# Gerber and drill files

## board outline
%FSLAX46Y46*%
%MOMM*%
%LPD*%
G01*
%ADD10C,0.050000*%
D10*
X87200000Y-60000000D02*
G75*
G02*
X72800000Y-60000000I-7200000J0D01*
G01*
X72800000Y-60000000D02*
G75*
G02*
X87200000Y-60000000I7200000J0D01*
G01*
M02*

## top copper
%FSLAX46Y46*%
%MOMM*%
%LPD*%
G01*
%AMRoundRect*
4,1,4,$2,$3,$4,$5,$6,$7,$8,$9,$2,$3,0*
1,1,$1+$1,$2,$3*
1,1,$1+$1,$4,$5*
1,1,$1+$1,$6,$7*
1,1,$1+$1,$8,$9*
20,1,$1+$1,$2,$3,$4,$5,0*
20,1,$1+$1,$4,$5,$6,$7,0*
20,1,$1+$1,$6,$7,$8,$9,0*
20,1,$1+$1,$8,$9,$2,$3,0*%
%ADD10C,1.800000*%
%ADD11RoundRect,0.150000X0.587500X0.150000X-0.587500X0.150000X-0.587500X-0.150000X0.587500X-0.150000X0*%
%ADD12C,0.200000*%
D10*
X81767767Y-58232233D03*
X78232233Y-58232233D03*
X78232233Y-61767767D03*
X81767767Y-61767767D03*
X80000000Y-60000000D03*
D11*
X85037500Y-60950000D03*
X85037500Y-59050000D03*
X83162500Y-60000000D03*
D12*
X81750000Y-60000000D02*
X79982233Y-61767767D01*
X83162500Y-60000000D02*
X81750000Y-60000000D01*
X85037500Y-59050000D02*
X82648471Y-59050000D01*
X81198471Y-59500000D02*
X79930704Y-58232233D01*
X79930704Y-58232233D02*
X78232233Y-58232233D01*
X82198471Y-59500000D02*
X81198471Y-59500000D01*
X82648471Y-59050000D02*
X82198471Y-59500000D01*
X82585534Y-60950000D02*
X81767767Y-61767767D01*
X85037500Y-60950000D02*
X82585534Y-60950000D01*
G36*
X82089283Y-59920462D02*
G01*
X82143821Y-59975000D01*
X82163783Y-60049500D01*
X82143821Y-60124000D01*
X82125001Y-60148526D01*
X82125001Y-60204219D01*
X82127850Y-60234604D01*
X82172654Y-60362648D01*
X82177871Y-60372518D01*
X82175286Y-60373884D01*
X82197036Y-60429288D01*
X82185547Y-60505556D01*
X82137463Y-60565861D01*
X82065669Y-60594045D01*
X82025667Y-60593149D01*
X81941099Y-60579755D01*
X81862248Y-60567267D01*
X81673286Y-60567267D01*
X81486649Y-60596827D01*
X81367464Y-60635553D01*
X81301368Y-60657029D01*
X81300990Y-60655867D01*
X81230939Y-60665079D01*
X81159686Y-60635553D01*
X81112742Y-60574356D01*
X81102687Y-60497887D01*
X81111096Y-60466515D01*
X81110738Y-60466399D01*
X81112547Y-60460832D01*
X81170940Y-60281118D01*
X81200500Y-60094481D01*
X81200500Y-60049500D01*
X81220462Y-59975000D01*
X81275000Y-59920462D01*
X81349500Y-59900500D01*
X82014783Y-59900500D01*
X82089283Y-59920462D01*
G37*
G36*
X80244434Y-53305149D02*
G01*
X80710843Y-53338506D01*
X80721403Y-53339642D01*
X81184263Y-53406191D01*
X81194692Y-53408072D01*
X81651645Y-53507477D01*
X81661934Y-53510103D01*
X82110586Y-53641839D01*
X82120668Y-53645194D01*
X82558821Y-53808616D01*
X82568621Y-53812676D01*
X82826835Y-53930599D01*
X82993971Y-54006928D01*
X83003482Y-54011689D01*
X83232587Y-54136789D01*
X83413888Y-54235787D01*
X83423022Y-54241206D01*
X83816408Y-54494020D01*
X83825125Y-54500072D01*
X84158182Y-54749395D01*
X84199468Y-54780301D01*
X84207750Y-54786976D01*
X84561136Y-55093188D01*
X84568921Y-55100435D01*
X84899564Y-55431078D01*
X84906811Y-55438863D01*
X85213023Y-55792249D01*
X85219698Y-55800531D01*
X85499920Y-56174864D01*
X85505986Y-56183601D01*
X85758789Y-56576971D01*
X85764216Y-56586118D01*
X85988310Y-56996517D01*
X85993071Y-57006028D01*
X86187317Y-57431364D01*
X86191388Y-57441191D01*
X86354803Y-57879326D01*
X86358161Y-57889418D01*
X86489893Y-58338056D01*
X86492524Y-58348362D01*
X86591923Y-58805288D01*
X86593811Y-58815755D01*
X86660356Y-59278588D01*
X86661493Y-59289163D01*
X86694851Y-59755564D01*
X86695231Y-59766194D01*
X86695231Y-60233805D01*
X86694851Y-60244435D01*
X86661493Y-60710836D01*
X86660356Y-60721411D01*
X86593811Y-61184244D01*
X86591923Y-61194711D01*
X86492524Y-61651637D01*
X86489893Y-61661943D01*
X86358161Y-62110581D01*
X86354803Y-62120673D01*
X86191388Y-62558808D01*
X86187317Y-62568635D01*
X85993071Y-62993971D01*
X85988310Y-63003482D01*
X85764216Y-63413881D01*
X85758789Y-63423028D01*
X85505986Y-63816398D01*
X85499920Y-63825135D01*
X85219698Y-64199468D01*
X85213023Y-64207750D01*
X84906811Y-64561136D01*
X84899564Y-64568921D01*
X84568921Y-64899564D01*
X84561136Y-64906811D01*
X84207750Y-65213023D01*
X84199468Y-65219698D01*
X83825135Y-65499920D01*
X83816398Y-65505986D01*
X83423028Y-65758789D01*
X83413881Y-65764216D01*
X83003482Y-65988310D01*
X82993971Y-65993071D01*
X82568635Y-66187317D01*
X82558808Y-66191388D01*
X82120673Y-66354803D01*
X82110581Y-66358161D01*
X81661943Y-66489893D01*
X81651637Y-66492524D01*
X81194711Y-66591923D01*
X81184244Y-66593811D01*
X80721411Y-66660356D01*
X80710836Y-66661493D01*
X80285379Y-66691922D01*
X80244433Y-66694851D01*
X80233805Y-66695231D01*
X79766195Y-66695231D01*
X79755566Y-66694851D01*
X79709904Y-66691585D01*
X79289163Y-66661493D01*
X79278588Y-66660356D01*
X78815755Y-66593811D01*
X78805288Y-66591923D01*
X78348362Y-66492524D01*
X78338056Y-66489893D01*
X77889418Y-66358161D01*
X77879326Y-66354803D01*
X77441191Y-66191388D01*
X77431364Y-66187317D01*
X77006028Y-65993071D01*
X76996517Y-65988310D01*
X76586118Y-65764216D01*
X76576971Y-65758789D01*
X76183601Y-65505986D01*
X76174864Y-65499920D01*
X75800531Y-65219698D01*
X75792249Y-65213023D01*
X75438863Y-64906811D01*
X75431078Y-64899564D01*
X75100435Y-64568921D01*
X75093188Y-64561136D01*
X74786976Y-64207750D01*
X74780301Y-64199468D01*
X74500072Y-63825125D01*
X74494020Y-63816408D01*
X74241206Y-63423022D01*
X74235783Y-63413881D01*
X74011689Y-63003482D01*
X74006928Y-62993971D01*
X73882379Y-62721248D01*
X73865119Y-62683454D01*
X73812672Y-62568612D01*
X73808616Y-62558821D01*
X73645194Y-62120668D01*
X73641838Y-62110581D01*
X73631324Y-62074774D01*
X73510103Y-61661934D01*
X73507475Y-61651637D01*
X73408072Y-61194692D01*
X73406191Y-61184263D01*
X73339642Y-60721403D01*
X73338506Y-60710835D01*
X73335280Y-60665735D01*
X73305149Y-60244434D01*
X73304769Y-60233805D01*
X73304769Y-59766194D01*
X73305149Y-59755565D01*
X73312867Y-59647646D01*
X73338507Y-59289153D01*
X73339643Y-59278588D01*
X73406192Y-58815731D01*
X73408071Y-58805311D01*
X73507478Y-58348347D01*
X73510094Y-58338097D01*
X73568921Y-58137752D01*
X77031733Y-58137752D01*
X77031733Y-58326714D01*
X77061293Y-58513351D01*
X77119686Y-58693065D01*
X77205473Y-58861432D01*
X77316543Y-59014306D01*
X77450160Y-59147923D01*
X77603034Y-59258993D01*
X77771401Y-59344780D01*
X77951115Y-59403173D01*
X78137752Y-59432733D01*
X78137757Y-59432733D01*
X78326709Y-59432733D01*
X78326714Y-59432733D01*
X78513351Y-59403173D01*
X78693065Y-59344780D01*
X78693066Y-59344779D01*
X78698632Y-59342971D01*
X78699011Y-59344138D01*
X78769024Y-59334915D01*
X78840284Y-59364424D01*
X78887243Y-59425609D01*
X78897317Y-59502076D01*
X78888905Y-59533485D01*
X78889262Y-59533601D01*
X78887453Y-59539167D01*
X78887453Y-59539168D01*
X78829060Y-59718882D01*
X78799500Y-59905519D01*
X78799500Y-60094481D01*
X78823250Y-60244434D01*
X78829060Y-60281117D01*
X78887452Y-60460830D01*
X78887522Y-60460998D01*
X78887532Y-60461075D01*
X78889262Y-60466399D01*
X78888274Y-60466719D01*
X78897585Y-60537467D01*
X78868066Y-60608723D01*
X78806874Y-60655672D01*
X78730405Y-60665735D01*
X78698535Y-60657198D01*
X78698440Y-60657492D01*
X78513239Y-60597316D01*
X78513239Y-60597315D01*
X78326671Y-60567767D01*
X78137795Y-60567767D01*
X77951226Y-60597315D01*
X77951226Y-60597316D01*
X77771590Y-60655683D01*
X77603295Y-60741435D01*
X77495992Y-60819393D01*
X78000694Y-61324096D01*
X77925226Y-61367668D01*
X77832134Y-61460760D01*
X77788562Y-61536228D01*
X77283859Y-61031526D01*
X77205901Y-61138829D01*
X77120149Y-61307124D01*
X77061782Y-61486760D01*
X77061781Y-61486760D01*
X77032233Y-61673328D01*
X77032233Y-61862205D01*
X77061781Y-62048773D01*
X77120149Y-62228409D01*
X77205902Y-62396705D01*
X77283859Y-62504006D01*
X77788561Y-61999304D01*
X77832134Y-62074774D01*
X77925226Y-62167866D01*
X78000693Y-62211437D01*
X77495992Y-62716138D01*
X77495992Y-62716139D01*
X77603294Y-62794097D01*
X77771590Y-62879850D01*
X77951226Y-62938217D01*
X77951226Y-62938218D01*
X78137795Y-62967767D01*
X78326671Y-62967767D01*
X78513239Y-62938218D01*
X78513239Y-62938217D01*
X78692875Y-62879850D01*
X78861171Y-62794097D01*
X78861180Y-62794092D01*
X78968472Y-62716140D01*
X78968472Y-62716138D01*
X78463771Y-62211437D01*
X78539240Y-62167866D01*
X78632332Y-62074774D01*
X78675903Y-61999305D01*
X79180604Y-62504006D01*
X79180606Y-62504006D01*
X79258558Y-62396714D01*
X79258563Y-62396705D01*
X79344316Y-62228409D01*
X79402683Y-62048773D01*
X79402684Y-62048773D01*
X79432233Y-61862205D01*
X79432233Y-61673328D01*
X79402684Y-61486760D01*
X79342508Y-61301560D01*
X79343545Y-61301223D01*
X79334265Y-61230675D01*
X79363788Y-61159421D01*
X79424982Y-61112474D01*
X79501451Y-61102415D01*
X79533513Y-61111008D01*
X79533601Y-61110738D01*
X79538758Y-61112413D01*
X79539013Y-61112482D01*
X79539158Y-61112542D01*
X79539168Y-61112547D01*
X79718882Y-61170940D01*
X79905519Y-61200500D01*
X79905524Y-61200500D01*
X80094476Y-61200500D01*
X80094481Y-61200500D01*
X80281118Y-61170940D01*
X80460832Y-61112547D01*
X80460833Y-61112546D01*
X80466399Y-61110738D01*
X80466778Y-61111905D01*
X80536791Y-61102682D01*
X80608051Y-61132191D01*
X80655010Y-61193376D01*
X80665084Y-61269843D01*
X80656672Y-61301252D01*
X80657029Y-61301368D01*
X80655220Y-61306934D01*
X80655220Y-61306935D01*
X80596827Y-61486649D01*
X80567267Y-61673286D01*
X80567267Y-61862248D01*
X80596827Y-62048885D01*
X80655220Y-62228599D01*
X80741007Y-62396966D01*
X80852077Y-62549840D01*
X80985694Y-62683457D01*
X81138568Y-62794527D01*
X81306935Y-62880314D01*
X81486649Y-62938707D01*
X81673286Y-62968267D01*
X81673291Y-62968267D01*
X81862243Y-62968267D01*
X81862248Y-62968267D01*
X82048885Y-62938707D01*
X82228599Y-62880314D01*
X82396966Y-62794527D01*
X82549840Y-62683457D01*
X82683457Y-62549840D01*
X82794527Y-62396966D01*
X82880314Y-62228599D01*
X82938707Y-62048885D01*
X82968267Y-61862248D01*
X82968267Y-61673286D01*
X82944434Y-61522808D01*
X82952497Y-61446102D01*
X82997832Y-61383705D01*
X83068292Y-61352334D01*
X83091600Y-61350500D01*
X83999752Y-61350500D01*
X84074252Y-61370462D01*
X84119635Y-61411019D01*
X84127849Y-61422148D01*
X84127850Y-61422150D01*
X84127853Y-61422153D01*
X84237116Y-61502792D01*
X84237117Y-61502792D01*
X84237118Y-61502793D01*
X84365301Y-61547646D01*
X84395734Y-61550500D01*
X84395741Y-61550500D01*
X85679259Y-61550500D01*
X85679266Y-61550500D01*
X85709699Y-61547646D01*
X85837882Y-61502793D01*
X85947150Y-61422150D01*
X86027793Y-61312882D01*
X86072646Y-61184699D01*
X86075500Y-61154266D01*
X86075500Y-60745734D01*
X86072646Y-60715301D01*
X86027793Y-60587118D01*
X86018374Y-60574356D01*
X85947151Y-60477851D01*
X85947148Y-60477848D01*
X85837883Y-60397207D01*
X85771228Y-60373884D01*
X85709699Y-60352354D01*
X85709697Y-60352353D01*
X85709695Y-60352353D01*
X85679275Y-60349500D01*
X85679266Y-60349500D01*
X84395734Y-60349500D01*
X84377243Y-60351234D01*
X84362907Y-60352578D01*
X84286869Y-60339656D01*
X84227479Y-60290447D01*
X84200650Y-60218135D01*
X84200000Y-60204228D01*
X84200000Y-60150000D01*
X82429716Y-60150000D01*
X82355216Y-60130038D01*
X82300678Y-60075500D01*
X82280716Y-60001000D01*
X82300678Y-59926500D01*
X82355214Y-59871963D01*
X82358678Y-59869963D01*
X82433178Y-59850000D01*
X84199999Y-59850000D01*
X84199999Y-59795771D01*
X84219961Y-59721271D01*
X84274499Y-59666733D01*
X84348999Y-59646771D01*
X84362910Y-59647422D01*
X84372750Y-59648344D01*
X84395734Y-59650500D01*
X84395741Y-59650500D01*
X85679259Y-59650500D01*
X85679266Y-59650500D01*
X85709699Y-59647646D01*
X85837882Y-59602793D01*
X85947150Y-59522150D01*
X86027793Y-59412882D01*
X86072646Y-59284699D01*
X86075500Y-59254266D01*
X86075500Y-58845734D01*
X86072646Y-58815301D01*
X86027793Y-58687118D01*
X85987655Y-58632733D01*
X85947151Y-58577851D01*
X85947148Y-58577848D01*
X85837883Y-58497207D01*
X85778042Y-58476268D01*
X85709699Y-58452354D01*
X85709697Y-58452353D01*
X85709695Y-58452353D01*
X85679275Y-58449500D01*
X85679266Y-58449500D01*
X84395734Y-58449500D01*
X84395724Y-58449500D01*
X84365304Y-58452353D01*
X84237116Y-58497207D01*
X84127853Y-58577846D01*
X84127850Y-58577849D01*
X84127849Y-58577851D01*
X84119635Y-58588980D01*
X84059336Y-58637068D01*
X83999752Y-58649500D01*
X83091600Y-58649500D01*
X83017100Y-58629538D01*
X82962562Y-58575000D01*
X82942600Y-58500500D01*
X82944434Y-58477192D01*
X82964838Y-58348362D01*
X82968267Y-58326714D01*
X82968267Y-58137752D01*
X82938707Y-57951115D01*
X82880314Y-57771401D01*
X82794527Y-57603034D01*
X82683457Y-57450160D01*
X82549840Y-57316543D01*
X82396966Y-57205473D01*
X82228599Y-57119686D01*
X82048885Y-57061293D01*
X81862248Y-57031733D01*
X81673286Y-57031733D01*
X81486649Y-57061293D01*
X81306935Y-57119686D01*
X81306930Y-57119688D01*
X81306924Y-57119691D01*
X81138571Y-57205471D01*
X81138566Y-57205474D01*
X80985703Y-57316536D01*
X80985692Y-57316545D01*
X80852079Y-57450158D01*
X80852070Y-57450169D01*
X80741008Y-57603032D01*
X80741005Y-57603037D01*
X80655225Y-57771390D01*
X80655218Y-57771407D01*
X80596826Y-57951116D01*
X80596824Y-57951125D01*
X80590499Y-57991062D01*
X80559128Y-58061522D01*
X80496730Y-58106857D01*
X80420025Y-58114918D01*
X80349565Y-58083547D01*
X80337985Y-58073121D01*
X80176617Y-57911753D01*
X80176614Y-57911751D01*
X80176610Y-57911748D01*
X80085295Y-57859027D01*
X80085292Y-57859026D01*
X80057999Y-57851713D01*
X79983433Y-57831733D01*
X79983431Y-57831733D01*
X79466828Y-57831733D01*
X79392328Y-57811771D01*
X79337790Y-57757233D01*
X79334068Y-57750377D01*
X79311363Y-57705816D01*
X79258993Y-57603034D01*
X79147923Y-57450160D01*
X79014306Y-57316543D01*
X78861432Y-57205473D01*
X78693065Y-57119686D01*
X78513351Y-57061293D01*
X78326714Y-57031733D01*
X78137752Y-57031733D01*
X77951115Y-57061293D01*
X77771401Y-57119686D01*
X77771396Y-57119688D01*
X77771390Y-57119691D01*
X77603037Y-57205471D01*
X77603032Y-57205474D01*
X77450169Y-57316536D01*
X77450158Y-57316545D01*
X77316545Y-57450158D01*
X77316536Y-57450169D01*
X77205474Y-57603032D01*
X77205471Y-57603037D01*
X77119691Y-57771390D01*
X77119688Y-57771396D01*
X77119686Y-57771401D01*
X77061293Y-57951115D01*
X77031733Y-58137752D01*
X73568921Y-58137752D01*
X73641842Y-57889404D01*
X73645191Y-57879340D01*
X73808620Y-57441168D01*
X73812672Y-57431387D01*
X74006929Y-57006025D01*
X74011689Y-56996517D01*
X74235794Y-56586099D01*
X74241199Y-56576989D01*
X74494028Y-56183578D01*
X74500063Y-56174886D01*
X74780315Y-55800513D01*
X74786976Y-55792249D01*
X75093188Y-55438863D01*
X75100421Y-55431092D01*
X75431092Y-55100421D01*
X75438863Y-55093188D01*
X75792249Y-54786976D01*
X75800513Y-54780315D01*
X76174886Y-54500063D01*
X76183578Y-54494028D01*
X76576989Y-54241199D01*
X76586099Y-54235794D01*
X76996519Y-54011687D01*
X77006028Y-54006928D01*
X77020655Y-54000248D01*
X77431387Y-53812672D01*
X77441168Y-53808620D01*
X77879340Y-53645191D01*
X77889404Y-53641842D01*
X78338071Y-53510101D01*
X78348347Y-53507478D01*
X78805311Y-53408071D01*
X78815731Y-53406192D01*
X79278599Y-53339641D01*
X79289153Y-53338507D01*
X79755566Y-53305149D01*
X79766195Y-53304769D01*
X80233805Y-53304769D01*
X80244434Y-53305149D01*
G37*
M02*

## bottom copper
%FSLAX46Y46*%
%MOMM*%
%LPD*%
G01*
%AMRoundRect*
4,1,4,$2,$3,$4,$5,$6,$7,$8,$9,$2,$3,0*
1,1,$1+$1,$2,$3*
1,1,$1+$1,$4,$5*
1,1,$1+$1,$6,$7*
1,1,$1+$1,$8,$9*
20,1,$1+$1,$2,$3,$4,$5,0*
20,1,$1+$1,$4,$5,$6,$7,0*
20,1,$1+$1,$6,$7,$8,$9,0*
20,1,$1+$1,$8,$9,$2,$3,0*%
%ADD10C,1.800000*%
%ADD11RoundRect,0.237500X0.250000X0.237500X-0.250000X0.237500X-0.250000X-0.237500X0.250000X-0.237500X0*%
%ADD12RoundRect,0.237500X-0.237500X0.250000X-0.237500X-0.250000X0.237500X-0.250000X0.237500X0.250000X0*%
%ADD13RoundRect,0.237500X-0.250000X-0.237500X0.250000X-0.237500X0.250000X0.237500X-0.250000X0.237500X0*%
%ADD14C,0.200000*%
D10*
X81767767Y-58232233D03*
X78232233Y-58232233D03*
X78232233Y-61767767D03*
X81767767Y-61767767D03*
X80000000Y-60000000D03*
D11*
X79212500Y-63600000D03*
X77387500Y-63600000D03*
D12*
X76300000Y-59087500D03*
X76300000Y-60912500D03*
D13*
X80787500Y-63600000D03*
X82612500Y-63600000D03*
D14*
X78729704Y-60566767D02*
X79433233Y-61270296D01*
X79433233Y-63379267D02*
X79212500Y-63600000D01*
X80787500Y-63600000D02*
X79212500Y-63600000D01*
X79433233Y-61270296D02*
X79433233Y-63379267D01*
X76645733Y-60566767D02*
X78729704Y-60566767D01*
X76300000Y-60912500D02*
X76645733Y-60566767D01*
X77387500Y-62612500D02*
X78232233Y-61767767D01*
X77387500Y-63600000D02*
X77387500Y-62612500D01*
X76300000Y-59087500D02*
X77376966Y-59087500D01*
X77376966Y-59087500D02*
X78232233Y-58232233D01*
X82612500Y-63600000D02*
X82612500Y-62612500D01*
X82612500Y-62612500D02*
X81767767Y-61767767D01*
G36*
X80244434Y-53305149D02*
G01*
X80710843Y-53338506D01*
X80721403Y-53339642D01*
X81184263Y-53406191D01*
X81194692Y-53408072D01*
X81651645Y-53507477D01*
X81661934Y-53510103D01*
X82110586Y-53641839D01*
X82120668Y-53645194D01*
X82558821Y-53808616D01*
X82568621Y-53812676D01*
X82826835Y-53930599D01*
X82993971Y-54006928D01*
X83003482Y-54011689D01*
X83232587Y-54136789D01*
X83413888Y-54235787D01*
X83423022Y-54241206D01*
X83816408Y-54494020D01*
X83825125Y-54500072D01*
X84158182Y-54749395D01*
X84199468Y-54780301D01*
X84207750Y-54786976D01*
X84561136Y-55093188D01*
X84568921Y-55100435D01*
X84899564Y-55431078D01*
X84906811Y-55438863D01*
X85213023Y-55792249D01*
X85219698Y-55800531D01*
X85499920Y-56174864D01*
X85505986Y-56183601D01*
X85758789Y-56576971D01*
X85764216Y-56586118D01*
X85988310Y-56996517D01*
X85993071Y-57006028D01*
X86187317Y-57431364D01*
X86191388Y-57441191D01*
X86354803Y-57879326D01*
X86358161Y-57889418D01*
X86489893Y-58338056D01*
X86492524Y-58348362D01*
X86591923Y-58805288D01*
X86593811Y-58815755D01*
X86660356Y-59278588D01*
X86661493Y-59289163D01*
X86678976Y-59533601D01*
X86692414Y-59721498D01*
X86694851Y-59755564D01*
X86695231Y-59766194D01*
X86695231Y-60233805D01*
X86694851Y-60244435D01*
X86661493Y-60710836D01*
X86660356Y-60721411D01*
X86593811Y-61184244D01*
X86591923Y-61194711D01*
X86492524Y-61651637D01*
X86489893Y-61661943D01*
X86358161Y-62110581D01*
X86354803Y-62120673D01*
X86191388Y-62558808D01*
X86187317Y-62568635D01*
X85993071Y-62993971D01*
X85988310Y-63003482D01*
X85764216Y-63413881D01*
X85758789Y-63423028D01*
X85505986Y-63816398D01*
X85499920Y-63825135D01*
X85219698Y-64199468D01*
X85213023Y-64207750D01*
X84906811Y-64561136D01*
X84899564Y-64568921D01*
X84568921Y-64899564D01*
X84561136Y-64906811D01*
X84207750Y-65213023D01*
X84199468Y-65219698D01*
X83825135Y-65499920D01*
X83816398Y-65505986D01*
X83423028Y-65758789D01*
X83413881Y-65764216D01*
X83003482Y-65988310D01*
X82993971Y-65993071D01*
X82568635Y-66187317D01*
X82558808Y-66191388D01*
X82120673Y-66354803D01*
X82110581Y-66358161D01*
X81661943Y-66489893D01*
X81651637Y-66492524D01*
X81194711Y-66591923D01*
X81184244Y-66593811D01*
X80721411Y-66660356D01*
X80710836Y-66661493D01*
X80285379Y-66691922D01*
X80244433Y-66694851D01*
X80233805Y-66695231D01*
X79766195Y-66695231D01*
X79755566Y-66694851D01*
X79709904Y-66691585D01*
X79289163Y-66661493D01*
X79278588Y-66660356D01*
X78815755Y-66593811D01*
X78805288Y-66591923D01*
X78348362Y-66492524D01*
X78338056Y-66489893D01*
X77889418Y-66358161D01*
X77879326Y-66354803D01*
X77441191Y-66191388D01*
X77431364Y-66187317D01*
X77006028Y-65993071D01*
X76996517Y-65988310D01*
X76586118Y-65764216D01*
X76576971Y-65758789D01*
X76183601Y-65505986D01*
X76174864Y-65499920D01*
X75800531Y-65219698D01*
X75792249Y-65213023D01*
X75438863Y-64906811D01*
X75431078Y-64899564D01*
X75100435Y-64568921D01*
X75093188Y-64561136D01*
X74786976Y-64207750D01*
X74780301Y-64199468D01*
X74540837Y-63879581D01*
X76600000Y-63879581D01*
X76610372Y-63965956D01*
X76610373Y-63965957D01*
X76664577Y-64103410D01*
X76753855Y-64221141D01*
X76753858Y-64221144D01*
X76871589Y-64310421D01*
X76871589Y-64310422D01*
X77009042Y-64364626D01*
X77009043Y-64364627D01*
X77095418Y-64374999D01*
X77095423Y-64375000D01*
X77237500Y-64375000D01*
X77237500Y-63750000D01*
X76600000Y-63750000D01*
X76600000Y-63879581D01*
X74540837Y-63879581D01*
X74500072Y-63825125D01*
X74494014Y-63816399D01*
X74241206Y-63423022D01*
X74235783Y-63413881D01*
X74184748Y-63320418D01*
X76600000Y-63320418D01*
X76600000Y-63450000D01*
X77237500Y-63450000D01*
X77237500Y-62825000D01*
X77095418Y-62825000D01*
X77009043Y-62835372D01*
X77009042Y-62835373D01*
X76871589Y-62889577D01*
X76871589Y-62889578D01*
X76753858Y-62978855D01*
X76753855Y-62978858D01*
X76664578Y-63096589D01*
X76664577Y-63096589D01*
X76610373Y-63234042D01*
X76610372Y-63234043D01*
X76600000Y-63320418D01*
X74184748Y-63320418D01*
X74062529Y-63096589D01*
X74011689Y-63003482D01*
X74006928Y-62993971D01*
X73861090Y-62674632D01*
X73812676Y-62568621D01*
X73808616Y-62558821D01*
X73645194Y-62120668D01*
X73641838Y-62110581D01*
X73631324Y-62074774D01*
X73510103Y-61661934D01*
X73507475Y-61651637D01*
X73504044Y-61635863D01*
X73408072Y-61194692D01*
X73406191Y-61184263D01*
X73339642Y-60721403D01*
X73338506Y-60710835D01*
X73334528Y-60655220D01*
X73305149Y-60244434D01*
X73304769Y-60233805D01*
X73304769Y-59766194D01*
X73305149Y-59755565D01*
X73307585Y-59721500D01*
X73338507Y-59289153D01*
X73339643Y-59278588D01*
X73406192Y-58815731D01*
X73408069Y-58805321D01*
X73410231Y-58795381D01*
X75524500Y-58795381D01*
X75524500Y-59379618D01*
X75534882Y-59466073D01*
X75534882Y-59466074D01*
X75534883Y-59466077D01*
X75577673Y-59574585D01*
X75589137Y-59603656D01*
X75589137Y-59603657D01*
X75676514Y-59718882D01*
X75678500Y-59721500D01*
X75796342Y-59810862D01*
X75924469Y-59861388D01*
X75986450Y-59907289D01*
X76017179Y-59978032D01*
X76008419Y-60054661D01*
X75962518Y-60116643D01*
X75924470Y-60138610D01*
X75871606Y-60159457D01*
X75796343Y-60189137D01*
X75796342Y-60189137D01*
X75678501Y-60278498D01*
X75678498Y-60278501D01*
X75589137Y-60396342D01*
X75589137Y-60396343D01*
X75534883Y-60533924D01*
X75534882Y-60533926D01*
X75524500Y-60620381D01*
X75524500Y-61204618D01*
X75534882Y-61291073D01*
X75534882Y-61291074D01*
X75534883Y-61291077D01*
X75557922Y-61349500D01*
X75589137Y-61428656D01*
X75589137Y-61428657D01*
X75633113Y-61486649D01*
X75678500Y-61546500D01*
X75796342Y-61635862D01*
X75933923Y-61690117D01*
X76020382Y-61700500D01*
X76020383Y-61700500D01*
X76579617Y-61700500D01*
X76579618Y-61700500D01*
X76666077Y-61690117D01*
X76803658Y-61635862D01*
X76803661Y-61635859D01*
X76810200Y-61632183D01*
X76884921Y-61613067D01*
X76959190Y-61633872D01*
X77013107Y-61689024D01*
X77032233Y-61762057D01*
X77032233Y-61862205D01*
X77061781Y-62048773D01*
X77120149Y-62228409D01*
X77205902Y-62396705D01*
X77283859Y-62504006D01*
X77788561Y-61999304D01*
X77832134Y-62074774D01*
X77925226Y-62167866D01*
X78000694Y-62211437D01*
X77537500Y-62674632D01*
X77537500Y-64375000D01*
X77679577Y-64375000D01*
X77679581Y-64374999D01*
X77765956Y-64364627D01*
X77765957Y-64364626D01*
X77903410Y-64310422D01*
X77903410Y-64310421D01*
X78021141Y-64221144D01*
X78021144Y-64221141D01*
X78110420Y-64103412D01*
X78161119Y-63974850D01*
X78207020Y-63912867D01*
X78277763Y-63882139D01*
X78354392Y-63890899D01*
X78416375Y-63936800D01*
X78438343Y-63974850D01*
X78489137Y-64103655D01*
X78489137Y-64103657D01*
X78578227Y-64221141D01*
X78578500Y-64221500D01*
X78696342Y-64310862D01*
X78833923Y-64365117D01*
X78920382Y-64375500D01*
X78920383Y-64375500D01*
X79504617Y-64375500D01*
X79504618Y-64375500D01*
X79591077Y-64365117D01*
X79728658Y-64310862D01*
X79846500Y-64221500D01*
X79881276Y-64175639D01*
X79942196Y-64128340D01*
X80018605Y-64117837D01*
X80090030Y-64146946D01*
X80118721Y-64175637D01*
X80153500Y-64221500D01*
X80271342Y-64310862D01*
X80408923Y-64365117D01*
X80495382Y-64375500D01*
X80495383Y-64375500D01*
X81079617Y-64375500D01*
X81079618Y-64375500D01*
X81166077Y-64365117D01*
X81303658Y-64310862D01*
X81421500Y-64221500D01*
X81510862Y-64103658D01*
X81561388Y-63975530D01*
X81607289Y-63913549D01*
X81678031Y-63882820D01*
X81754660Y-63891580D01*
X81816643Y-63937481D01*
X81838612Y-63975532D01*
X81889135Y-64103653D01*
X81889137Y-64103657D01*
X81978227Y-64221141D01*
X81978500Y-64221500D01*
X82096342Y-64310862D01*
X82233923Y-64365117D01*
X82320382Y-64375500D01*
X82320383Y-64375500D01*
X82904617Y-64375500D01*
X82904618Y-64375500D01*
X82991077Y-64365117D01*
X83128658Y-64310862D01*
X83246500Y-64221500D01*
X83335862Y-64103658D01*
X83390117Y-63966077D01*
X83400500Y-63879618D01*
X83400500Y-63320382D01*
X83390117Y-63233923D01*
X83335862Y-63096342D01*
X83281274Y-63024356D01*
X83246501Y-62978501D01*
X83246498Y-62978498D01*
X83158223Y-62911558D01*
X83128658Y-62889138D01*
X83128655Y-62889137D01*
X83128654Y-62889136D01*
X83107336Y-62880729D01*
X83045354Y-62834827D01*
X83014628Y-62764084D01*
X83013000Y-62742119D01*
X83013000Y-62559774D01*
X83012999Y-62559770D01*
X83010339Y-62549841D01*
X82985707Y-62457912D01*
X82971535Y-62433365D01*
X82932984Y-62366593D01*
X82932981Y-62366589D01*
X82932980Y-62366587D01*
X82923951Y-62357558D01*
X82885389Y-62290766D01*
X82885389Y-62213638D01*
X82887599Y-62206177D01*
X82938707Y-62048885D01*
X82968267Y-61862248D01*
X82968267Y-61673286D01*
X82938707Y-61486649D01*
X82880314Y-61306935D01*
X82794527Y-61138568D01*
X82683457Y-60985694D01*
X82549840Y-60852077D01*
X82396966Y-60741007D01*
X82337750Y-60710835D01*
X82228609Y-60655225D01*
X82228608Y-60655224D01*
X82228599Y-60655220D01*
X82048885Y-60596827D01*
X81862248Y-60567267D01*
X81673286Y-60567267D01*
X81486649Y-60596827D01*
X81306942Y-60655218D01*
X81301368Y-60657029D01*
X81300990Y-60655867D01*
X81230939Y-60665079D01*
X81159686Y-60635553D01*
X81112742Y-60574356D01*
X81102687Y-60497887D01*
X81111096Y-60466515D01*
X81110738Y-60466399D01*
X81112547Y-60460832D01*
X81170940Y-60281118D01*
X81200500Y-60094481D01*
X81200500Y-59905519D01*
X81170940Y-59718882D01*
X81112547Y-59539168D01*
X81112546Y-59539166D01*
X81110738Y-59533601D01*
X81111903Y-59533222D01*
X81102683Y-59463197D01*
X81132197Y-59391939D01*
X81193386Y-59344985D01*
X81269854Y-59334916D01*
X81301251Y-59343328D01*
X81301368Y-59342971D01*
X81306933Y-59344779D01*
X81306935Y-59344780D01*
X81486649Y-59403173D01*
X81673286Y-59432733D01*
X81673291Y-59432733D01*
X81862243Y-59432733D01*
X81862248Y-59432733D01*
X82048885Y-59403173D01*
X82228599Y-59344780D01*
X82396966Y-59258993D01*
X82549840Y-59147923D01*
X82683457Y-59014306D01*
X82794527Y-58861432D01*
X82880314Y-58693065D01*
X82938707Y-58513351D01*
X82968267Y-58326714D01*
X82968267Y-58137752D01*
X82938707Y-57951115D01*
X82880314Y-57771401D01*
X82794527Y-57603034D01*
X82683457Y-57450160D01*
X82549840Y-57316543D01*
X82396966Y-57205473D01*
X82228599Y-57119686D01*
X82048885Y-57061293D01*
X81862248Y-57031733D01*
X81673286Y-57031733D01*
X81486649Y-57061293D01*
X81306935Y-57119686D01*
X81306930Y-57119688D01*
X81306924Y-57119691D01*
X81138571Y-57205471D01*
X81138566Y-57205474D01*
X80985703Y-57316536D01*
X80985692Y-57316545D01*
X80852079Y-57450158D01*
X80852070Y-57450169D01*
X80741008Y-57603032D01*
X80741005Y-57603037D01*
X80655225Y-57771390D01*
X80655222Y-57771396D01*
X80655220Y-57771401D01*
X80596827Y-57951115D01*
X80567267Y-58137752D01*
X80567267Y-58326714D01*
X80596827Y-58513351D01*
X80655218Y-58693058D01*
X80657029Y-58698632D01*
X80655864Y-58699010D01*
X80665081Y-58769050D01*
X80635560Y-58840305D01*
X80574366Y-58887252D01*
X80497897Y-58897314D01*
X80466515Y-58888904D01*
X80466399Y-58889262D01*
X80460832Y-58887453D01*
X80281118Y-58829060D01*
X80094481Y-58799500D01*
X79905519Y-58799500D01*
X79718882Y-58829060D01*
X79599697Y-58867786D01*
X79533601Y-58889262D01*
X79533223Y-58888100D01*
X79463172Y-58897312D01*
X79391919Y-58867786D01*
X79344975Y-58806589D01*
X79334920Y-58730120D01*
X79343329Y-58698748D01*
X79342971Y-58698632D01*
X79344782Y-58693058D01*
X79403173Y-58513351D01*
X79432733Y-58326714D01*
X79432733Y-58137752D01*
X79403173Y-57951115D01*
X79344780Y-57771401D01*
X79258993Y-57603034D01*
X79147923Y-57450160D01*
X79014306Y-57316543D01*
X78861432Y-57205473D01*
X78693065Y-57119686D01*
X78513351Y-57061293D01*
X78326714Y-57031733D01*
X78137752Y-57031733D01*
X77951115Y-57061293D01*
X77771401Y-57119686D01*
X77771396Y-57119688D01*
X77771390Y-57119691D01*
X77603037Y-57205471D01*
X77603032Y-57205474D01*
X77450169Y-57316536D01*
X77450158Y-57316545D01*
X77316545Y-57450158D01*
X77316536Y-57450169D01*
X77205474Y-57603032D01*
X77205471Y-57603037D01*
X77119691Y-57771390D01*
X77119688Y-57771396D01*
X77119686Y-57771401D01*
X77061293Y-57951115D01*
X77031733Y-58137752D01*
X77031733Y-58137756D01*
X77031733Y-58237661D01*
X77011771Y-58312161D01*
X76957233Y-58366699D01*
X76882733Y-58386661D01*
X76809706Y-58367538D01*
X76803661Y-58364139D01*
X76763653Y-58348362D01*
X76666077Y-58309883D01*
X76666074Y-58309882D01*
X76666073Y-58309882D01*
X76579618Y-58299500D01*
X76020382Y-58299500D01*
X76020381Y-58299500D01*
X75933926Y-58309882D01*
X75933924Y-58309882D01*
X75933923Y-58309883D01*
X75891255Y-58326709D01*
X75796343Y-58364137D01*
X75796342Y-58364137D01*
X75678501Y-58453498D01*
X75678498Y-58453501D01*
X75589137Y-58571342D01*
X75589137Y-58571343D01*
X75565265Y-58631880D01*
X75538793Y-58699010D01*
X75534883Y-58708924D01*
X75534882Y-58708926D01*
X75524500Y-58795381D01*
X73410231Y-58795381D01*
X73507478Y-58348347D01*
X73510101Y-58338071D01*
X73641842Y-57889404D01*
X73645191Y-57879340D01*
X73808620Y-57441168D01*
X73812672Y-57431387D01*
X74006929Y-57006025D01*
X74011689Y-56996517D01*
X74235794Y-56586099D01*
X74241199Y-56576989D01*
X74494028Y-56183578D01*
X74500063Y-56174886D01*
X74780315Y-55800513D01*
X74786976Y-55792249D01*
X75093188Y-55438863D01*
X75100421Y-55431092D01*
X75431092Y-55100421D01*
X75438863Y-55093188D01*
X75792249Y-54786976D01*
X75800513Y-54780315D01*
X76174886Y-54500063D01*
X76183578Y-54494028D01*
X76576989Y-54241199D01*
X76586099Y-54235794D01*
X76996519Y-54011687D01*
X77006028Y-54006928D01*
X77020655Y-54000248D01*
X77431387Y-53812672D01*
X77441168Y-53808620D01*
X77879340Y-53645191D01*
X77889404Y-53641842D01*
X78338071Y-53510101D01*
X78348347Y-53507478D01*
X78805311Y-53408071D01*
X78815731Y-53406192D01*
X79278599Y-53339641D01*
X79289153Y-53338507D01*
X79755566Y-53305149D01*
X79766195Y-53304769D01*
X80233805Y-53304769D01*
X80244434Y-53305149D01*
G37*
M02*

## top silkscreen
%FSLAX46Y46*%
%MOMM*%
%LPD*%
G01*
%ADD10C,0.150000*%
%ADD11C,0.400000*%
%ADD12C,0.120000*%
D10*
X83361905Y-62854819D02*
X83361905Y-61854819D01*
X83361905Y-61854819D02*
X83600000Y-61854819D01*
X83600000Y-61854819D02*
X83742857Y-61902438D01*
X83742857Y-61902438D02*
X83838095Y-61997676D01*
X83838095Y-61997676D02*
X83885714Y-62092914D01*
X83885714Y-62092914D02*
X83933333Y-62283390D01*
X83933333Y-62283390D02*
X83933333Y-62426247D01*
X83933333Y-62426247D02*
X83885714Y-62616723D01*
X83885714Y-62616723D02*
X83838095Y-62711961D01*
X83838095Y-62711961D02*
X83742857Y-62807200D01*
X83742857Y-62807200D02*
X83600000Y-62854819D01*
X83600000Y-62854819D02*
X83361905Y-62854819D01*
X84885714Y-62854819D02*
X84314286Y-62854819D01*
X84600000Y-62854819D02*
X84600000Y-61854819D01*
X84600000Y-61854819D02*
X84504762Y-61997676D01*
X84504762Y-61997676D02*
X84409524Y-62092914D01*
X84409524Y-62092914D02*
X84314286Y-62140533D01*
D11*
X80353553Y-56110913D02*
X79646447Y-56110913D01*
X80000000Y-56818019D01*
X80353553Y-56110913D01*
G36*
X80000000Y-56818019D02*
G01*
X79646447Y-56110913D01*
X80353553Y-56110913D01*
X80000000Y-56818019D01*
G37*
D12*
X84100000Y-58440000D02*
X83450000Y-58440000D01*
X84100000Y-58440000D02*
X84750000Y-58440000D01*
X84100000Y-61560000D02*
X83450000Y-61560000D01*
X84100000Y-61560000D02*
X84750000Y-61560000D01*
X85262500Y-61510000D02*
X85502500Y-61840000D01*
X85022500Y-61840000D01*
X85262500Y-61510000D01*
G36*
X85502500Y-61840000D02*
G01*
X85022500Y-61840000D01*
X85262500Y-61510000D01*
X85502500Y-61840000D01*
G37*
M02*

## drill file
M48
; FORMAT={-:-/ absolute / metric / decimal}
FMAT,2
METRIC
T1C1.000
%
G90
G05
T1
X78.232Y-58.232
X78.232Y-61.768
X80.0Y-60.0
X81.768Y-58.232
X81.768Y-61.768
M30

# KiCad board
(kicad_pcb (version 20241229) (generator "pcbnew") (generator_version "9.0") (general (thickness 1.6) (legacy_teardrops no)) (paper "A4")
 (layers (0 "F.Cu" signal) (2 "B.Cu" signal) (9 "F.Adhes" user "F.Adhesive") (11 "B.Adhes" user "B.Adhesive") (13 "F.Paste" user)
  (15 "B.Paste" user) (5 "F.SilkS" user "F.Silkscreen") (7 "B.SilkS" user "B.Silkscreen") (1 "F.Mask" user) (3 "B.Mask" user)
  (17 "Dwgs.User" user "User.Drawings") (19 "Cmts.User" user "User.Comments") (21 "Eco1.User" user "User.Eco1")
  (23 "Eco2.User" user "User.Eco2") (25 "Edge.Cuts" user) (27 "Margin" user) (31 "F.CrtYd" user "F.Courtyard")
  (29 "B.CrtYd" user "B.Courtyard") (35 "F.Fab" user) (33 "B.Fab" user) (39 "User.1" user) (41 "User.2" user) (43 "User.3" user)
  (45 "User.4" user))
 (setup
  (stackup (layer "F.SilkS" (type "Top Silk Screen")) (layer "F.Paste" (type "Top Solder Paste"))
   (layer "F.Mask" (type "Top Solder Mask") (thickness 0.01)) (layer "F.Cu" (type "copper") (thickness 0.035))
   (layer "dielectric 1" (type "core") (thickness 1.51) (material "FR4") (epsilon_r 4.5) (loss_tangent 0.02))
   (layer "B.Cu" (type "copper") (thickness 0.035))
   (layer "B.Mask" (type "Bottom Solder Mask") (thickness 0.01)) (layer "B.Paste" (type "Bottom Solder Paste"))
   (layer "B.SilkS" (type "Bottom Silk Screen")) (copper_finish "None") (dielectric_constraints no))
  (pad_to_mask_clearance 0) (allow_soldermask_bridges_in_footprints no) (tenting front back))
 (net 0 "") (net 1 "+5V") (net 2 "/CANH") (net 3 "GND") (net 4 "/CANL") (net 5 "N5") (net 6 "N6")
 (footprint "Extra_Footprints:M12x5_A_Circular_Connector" (layer "F.Cu") (at 80 60 45)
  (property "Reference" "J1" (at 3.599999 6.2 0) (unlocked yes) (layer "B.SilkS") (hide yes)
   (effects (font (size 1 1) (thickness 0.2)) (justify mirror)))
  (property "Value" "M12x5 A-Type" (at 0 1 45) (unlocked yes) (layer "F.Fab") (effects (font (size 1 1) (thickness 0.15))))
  (fp_poly (pts (xy 3 -2.5) (xy 2.5 -3) (xy 2.25 -2.25)) (stroke (width 0.4) (type solid)) (fill yes) (layer "F.SilkS"))
  (pad "1" thru_hole circle (at 2.5 0 45) (size 1.8 1.8) (drill 1) (layers "*.Cu" "*.Mask") (remove_unused_layers no) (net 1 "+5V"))
  (pad "2" thru_hole circle (at 0 -2.5 45) (size 1.8 1.8) (drill 1) (layers "*.Cu" "*.Mask") (remove_unused_layers no) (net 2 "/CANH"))
  (pad "3" thru_hole circle (at -2.5 0 45) (size 1.8 1.8) (drill 1) (layers "*.Cu" "*.Mask") (remove_unused_layers no) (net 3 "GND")
   (thermal_bridge_angle 0))
  (pad "4" thru_hole circle (at 0 2.5 45) (size 1.8 1.8) (drill 1) (layers "*.Cu" "*.Mask") (remove_unused_layers no) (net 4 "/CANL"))
  (pad "5" thru_hole circle (at 0 0 45) (size 1.8 1.8) (drill 1) (layers "*.Cu" "*.Mask") (remove_unused_layers no) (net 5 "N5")))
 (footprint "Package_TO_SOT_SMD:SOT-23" (layer "F.Cu") (at 84.1 60 180)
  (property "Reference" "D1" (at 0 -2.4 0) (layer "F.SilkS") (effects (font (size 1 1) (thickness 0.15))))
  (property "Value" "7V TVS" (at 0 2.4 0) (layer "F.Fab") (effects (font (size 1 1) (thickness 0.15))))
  (fp_line (start 0 1.56) (end 0.65 1.56) (stroke (width 0.12) (type solid)) (layer "F.SilkS"))
  (fp_line (start 0 1.56) (end -0.65 1.56) (stroke (width 0.12) (type solid)) (layer "F.SilkS"))
  (fp_line (start 0 -1.56) (end 0.65 -1.56) (stroke (width 0.12) (type solid)) (layer "F.SilkS"))
  (fp_line (start 0 -1.56) (end -0.65 -1.56) (stroke (width 0.12) (type solid)) (layer "F.SilkS"))
  (fp_poly (pts (xy -1.1625 -1.51) (xy -1.4025 -1.84) (xy -0.9225 -1.84)) (stroke (width 0.12) (type solid)) (fill yes) (layer "F.SilkS"))
  (pad "1" smd roundrect (at -0.9375 -0.95 180) (size 1.475 0.6) (layers "F.Cu" "F.Mask" "F.Paste") (roundrect_rratio 0.25) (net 4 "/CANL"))
  (pad "2" smd roundrect (at -0.9375 0.95 180) (size 1.475 0.6) (layers "F.Cu" "F.Mask" "F.Paste") (roundrect_rratio 0.25) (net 2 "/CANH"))
  (pad "3" smd roundrect (at 0.9375 0 180) (size 1.475 0.6) (layers "F.Cu" "F.Mask" "F.Paste") (roundrect_rratio 0.25) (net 3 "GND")))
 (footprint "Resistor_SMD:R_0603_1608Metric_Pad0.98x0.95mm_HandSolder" (layer "B.Cu") (at 78.3 63.6 180)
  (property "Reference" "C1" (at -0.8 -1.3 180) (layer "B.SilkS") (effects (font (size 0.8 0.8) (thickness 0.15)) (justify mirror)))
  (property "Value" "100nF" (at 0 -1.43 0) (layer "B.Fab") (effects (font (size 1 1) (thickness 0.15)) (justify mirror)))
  (pad "1" smd roundrect (at -0.9125 0 180) (size 0.975 0.95) (layers "B.Cu" "B.Mask" "B.Paste") (roundrect_rratio 0.25) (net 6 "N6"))
  (pad "2" smd roundrect (at 0.9125 0 180) (size 0.975 0.95) (layers "B.Cu" "B.Mask" "B.Paste") (roundrect_rratio 0.25) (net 3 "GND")))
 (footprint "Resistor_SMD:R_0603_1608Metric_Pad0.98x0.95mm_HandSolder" (layer "B.Cu") (at 76.3 60 -90)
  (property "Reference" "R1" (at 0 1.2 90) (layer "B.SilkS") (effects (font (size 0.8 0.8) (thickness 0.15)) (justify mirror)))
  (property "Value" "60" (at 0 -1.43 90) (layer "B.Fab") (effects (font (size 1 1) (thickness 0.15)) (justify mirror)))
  (pad "1" smd roundrect (at -0.9125 0 270) (size 0.975 0.95) (layers "B.Cu" "B.Mask" "B.Paste") (roundrect_rratio 0.25) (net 2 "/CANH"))
  (pad "2" smd roundrect (at 0.9125 0 270) (size 0.975 0.95) (layers "B.Cu" "B.Mask" "B.Paste") (roundrect_rratio 0.25) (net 6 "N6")))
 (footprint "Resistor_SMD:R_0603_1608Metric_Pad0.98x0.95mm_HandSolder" (layer "B.Cu") (at 81.7 63.6)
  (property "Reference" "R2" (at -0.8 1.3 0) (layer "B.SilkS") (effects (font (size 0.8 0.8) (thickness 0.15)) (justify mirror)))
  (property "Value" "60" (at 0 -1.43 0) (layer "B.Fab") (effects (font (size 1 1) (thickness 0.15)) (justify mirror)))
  (pad "1" smd roundrect (at -0.9125 0) (size 0.975 0.95) (layers "B.Cu" "B.Mask" "B.Paste") (roundrect_rratio 0.25) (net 6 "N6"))
  (pad "2" smd roundrect (at 0.9125 0) (size 0.975 0.95) (layers "B.Cu" "B.Mask" "B.Paste") (roundrect_rratio 0.25) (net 4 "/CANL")))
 (gr_circle (center 80 60) (end 87.2 60) (stroke (width 0.05) (type default)) (fill no) (layer "Edge.Cuts"))
 (segment (start 78.729704 60.566767) (end 79.433233 61.270296) (width 0.2) (layer "B.Cu") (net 6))
 (segment (start 79.433233 63.379267) (end 79.2125 63.6) (width 0.2) (layer "B.Cu") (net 6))
 (segment (start 80.7875 63.6) (end 79.2125 63.6) (width 0.2) (layer "B.Cu") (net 6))
 (segment (start 79.433233 61.270296) (end 79.433233 63.379267) (width 0.2) (layer "B.Cu") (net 6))
 (segment (start 76.645733 60.566767) (end 78.729704 60.566767) (width 0.2) (layer "B.Cu") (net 6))
 (segment (start 76.3 60.9125) (end 76.645733 60.566767) (width 0.2) (layer "B.Cu") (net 6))
 (segment (start 81.75 60) (end 79.982233 61.767767) (width 0.2) (layer "F.Cu") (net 3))
 (segment (start 83.1625 60) (end 81.75 60) (width 0.2) (layer "F.Cu") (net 3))
 (segment (start 77.3875 62.6125) (end 78.232233 61.767767) (width 0.2) (layer "B.Cu") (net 3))
 (segment (start 77.3875 63.6) (end 77.3875 62.6125) (width 0.2) (layer "B.Cu") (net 3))
 (segment (start 85.0375 59.05) (end 82.648471 59.05) (width 0.2) (layer "F.Cu") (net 2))
 (segment (start 81.198471 59.5) (end 79.930704 58.232233) (width 0.2) (layer "F.Cu") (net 2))
 (segment (start 79.930704 58.232233) (end 78.232233 58.232233) (width 0.2) (layer "F.Cu") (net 2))
 (segment (start 82.198471 59.5) (end 81.198471 59.5) (width 0.2) (layer "F.Cu") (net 2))
 (segment (start 82.648471 59.05) (end 82.198471 59.5) (width 0.2) (layer "F.Cu") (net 2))
 (segment (start 76.3 59.0875) (end 77.376966 59.0875) (width 0.2) (layer "B.Cu") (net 2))
 (segment (start 77.376966 59.0875) (end 78.232233 58.232233) (width 0.2) (layer "B.Cu") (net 2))
 (segment (start 82.585534 60.95) (end 81.767767 61.767767) (width 0.2) (layer "F.Cu") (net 4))
 (segment (start 85.0375 60.95) (end 82.585534 60.95) (width 0.2) (layer "F.Cu") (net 4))
 (segment (start 82.6125 63.6) (end 82.6125 62.6125) (width 0.2) (layer "B.Cu") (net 4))
 (segment (start 82.6125 62.6125) (end 81.767767 61.767767) (width 0.2) (layer "B.Cu") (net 4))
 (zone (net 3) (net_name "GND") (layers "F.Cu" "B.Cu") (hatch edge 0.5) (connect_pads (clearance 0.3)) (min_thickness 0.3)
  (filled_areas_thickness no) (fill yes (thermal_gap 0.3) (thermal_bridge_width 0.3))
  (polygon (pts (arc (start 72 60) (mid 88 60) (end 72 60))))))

